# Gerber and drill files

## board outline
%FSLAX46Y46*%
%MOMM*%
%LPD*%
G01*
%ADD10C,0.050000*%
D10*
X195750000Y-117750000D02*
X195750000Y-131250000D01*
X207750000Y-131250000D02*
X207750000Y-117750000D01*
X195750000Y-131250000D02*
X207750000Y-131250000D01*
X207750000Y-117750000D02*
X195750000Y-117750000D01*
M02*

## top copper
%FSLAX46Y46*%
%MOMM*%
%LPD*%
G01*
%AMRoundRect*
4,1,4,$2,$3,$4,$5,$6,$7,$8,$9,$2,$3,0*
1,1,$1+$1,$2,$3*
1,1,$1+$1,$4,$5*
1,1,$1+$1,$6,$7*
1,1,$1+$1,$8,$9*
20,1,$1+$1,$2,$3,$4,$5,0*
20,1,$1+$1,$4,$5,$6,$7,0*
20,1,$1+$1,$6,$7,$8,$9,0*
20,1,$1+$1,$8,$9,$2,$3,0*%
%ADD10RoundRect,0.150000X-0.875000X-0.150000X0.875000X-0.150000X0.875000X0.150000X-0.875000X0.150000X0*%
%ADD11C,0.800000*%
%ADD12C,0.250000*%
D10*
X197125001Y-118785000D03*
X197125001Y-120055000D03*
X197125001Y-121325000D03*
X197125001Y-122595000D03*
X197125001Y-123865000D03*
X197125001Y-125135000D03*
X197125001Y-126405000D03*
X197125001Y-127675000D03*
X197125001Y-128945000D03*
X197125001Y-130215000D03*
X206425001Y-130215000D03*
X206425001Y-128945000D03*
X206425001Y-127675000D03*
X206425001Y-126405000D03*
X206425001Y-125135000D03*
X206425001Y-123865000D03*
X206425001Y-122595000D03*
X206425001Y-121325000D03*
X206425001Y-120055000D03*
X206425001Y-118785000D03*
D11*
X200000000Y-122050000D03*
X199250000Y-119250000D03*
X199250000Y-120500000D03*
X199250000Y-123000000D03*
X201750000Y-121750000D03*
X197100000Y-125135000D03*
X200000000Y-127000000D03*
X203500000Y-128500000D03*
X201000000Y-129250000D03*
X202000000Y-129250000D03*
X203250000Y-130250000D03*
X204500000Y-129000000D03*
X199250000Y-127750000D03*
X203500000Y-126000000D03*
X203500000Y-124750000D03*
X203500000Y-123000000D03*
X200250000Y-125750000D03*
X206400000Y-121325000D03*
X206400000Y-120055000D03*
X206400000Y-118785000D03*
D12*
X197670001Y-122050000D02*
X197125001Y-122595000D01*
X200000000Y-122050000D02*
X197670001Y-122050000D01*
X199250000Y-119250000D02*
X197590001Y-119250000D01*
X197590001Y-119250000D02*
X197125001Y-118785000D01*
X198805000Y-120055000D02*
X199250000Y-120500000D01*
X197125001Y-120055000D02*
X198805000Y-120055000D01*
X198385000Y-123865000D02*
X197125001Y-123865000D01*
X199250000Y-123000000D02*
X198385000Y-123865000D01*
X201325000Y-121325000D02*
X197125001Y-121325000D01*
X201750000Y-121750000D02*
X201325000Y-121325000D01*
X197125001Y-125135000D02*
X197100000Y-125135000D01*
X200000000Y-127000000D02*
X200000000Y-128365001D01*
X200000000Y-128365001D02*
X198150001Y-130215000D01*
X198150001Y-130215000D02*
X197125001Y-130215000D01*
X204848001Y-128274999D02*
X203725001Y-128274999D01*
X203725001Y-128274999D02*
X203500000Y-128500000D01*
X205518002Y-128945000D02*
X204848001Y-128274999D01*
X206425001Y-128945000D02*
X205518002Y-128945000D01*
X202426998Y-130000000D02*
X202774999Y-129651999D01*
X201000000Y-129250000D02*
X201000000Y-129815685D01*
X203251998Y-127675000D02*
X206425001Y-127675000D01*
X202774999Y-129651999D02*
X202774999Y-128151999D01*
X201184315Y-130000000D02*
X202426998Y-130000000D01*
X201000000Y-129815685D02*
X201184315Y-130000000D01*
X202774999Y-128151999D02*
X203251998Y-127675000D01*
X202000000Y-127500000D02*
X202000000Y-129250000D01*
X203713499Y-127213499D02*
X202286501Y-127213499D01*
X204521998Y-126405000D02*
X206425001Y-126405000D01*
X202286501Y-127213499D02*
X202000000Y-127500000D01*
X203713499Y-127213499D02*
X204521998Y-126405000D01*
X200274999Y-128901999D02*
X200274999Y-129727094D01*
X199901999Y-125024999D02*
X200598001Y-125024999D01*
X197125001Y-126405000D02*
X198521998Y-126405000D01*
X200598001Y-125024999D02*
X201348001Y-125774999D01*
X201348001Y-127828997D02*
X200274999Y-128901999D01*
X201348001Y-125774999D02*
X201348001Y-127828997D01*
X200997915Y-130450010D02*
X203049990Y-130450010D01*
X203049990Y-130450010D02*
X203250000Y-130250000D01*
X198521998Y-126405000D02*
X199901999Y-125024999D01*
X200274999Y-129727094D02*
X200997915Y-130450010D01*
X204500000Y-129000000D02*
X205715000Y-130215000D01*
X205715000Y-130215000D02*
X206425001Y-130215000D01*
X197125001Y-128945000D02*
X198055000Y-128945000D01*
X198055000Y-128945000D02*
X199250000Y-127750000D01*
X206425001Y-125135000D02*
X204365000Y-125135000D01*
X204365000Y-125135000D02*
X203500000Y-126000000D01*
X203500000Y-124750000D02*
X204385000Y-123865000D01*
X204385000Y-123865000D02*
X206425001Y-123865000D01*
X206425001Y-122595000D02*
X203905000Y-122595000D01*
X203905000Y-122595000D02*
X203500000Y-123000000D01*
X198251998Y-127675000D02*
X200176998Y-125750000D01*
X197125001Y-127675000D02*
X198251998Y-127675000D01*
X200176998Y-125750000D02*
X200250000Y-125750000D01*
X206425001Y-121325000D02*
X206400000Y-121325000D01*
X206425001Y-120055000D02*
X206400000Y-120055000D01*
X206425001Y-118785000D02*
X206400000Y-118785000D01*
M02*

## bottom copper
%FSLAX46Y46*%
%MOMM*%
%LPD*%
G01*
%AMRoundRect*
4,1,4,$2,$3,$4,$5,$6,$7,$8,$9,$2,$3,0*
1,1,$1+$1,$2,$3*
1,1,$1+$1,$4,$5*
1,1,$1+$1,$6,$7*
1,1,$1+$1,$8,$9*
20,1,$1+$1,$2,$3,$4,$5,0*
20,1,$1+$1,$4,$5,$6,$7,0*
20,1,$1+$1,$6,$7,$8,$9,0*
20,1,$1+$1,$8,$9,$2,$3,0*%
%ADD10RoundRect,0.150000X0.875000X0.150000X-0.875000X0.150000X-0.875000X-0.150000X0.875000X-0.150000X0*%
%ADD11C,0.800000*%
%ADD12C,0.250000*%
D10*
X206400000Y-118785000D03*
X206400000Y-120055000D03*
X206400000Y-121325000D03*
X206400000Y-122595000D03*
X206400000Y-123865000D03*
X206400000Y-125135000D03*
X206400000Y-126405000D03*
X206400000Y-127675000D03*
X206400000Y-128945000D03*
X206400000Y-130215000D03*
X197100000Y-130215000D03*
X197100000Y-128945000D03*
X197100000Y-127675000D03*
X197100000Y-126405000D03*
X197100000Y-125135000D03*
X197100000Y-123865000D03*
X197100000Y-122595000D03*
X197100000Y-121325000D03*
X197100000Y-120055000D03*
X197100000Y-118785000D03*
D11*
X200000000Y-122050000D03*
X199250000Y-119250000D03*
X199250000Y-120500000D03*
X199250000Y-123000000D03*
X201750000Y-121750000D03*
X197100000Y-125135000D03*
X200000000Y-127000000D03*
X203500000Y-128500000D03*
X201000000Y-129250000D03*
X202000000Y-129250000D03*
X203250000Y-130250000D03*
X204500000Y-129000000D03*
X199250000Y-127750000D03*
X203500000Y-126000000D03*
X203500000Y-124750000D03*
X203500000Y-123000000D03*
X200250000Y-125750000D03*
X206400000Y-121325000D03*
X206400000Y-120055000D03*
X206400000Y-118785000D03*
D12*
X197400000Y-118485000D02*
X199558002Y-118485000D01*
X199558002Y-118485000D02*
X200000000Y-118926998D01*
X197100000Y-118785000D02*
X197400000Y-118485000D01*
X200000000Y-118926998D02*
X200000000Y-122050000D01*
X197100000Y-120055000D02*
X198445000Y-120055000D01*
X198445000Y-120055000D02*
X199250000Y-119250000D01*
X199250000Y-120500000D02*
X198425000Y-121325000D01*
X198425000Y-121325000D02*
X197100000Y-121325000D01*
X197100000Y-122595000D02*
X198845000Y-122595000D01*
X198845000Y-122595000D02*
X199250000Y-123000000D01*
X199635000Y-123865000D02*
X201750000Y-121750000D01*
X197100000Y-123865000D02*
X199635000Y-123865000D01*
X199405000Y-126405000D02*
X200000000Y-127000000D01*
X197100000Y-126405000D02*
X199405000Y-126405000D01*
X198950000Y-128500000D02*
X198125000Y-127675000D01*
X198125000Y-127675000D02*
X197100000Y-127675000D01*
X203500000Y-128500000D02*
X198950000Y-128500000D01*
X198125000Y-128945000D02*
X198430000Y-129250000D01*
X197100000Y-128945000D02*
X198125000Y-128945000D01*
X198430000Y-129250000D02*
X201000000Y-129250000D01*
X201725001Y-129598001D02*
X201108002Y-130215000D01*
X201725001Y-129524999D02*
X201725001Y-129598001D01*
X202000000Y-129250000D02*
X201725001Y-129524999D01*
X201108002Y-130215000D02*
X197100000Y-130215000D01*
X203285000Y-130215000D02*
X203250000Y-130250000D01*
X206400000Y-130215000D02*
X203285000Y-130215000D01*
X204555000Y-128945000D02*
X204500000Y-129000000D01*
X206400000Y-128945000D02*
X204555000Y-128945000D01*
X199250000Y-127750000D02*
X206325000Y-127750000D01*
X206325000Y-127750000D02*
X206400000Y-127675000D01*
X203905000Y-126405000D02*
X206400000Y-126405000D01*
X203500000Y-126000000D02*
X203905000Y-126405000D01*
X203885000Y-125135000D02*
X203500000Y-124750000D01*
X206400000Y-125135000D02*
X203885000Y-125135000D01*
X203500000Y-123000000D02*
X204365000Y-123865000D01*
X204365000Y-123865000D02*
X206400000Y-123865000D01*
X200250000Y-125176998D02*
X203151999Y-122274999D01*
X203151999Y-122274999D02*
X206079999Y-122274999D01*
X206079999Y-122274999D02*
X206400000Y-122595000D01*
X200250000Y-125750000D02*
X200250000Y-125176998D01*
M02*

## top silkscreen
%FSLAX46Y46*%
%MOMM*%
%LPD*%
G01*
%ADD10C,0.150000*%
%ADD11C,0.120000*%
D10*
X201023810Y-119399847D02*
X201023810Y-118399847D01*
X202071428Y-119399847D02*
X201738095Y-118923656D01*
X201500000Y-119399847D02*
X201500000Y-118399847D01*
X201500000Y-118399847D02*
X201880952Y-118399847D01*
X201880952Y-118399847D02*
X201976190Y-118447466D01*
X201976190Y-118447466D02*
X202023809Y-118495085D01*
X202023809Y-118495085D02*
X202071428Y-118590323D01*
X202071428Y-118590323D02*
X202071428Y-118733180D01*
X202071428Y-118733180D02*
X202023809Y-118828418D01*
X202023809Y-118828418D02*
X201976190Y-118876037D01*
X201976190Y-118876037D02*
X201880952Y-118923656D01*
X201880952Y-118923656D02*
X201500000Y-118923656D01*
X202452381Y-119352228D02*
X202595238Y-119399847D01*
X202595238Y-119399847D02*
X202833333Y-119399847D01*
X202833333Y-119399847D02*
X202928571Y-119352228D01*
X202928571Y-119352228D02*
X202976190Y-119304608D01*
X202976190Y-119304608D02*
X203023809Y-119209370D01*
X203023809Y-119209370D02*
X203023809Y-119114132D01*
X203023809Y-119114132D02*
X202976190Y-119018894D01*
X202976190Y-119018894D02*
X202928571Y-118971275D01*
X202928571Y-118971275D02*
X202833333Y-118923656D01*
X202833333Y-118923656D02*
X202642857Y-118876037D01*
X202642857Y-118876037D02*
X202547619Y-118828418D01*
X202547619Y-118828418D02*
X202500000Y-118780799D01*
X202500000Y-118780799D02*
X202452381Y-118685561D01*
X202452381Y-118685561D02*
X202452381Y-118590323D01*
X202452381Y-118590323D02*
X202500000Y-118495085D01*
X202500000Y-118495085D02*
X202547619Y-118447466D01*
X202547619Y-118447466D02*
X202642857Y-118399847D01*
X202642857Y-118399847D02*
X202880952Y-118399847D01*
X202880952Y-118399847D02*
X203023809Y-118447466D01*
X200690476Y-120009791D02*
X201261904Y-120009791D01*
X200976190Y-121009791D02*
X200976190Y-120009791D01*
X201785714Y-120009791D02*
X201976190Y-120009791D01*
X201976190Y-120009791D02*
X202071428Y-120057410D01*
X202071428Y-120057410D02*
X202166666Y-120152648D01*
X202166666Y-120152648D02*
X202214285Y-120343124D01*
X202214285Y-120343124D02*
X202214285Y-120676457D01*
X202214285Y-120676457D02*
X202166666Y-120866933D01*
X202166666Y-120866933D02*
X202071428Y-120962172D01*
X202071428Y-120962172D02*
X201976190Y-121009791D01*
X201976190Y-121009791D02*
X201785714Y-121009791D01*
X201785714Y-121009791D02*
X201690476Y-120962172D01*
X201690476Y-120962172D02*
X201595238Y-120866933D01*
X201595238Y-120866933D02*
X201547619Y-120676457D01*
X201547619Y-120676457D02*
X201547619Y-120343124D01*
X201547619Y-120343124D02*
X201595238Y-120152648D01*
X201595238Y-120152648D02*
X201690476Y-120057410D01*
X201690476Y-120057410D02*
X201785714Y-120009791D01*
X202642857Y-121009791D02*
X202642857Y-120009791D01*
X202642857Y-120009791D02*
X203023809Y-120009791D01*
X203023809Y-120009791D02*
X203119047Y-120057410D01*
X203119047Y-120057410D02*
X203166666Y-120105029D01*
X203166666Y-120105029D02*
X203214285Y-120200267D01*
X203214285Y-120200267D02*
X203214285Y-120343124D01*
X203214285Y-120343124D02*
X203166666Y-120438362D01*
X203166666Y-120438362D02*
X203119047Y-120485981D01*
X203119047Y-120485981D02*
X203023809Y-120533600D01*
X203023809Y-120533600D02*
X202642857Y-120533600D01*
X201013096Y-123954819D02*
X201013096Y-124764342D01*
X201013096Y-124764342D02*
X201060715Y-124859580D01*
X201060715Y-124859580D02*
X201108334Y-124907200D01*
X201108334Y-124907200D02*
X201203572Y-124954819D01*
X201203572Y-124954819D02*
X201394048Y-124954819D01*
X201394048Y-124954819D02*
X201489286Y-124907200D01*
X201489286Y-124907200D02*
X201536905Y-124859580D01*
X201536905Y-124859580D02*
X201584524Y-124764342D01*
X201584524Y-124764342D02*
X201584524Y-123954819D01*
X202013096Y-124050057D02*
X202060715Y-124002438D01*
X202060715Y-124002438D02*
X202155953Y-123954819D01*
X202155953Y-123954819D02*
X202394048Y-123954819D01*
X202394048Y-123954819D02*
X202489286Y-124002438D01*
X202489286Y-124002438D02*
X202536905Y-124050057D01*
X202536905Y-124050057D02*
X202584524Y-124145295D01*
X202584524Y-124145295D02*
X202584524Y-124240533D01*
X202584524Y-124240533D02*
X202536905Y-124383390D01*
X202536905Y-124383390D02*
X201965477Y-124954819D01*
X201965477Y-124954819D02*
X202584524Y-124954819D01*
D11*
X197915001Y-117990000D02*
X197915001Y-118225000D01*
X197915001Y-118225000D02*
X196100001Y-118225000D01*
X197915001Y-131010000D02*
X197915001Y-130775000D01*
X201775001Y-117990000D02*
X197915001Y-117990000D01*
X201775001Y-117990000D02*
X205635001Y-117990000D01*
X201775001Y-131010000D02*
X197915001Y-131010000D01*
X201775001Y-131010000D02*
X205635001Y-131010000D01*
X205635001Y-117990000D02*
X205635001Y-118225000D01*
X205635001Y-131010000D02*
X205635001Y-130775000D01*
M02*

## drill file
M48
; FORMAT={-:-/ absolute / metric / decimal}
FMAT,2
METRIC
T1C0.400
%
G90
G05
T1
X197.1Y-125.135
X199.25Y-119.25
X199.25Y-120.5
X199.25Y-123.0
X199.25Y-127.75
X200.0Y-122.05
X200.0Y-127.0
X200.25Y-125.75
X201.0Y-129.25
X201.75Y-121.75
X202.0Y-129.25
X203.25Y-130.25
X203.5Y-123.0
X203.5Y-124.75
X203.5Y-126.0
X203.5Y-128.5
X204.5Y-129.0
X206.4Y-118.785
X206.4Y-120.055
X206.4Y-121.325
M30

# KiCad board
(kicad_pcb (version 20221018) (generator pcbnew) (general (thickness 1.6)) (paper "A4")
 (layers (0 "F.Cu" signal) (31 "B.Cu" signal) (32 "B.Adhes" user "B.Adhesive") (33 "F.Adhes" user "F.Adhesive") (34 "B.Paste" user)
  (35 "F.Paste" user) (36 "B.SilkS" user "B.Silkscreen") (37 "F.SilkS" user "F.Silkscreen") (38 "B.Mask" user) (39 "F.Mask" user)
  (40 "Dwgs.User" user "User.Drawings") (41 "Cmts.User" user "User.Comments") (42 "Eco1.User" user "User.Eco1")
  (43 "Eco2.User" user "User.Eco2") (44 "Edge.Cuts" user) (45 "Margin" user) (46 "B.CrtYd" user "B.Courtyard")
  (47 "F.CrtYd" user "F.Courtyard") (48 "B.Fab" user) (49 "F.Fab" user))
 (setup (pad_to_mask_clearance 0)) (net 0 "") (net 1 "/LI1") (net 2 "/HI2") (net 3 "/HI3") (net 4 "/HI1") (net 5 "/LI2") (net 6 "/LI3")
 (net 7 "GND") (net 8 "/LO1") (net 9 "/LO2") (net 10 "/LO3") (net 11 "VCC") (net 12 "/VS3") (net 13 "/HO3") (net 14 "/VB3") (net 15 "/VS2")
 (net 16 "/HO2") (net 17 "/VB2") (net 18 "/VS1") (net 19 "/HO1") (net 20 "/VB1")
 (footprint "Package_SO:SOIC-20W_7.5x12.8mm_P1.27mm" (layer "F.Cu") (at 201.775001 124.5)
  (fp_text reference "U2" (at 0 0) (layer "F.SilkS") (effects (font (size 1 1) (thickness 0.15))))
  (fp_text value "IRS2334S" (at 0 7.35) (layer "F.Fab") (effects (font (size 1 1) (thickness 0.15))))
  (fp_line (start -3.86 -6.51) (end -3.86 -6.275) (stroke (width 0.12) (type solid)) (layer "F.SilkS"))
  (fp_line (start -3.86 -6.275) (end -5.675 -6.275) (stroke (width 0.12) (type solid)) (layer "F.SilkS"))
  (fp_line (start -3.86 6.51) (end -3.86 6.275) (stroke (width 0.12) (type solid)) (layer "F.SilkS"))
  (fp_line (start 0 -6.51) (end -3.86 -6.51) (stroke (width 0.12) (type solid)) (layer "F.SilkS"))
  (fp_line (start 0 -6.51) (end 3.86 -6.51) (stroke (width 0.12) (type solid)) (layer "F.SilkS"))
  (fp_line (start 0 6.51) (end -3.86 6.51) (stroke (width 0.12) (type solid)) (layer "F.SilkS"))
  (fp_line (start 0 6.51) (end 3.86 6.51) (stroke (width 0.12) (type solid)) (layer "F.SilkS"))
  (fp_line (start 3.86 -6.51) (end 3.86 -6.275) (stroke (width 0.12) (type solid)) (layer "F.SilkS"))
  (fp_line (start 3.86 6.51) (end 3.86 6.275) (stroke (width 0.12) (type solid)) (layer "F.SilkS"))
  (pad "1" smd roundrect (at -4.65 -5.715) (size 2.05 0.6) (layers "F.Cu" "F.Paste" "F.Mask") (roundrect_rratio 0.25) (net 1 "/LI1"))
  (pad "2" smd roundrect (at -4.65 -4.445) (size 2.05 0.6) (layers "F.Cu" "F.Paste" "F.Mask") (roundrect_rratio 0.25) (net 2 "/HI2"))
  (pad "3" smd roundrect (at -4.65 -3.175) (size 2.05 0.6) (layers "F.Cu" "F.Paste" "F.Mask") (roundrect_rratio 0.25) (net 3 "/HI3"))
  (pad "4" smd roundrect (at -4.65 -1.905) (size 2.05 0.6) (layers "F.Cu" "F.Paste" "F.Mask") (roundrect_rratio 0.25) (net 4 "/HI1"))
  (pad "5" smd roundrect (at -4.65 -0.635) (size 2.05 0.6) (layers "F.Cu" "F.Paste" "F.Mask") (roundrect_rratio 0.25) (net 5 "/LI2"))
  (pad "6" smd roundrect (at -4.65 0.635) (size 2.05 0.6) (layers "F.Cu" "F.Paste" "F.Mask") (roundrect_rratio 0.25) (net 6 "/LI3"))
  (pad "7" smd roundrect (at -4.65 1.905) (size 2.05 0.6) (layers "F.Cu" "F.Paste" "F.Mask") (roundrect_rratio 0.25) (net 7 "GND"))
  (pad "8" smd roundrect (at -4.65 3.175) (size 2.05 0.6) (layers "F.Cu" "F.Paste" "F.Mask") (roundrect_rratio 0.25) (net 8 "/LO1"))
  (pad "9" smd roundrect (at -4.65 4.445) (size 2.05 0.6) (layers "F.Cu" "F.Paste" "F.Mask") (roundrect_rratio 0.25) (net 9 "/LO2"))
  (pad "10" smd roundrect (at -4.65 5.715) (size 2.05 0.6) (layers "F.Cu" "F.Paste" "F.Mask") (roundrect_rratio 0.25) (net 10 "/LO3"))
  (pad "11" smd roundrect (at 4.65 5.715) (size 2.05 0.6) (layers "F.Cu" "F.Paste" "F.Mask") (roundrect_rratio 0.25) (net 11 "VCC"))
  (pad "12" smd roundrect (at 4.65 4.445) (size 2.05 0.6) (layers "F.Cu" "F.Paste" "F.Mask") (roundrect_rratio 0.25) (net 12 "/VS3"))
  (pad "13" smd roundrect (at 4.65 3.175) (size 2.05 0.6) (layers "F.Cu" "F.Paste" "F.Mask") (roundrect_rratio 0.25) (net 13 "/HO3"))
  (pad "14" smd roundrect (at 4.65 1.905) (size 2.05 0.6) (layers "F.Cu" "F.Paste" "F.Mask") (roundrect_rratio 0.25) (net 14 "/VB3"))
  (pad "15" smd roundrect (at 4.65 0.635) (size 2.05 0.6) (layers "F.Cu" "F.Paste" "F.Mask") (roundrect_rratio 0.25) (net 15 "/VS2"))
  (pad "16" smd roundrect (at 4.65 -0.635) (size 2.05 0.6) (layers "F.Cu" "F.Paste" "F.Mask") (roundrect_rratio 0.25) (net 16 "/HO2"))
  (pad "17" smd roundrect (at 4.65 -1.905) (size 2.05 0.6) (layers "F.Cu" "F.Paste" "F.Mask") (roundrect_rratio 0.25) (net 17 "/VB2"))
  (pad "18" smd roundrect (at 4.65 -3.175) (size 2.05 0.6) (layers "F.Cu" "F.Paste" "F.Mask") (roundrect_rratio 0.25) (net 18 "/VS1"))
  (pad "19" smd roundrect (at 4.65 -4.445) (size 2.05 0.6) (layers "F.Cu" "F.Paste" "F.Mask") (roundrect_rratio 0.25) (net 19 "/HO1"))
  (pad "20" smd roundrect (at 4.65 -5.715) (size 2.05 0.6) (layers "F.Cu" "F.Paste" "F.Mask") (roundrect_rratio 0.25) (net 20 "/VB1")))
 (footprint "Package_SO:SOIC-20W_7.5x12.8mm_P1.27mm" (layer "B.Cu") (at 201.75 124.5 180)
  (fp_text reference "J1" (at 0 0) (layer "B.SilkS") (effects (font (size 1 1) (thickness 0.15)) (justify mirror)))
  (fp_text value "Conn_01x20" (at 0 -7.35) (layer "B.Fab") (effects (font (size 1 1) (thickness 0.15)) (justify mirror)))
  (pad "1" smd roundrect (at -4.65 5.715 180) (size 2.05 0.6) (layers "B.Cu" "B.Paste" "B.Mask") (roundrect_rratio 0.25) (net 20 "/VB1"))
  (pad "2" smd roundrect (at -4.65 4.445 180) (size 2.05 0.6) (layers "B.Cu" "B.Paste" "B.Mask") (roundrect_rratio 0.25) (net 19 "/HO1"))
  (pad "3" smd roundrect (at -4.65 3.175 180) (size 2.05 0.6) (layers "B.Cu" "B.Paste" "B.Mask") (roundrect_rratio 0.25) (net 18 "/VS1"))
  (pad "4" smd roundrect (at -4.65 1.905 180) (size 2.05 0.6) (layers "B.Cu" "B.Paste" "B.Mask") (roundrect_rratio 0.25) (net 8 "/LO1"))
  (pad "5" smd roundrect (at -4.65 0.635 180) (size 2.05 0.6) (layers "B.Cu" "B.Paste" "B.Mask") (roundrect_rratio 0.25) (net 17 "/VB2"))
  (pad "6" smd roundrect (at -4.65 -0.635 180) (size 2.05 0.6) (layers "B.Cu" "B.Paste" "B.Mask") (roundrect_rratio 0.25) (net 16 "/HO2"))
  (pad "7" smd roundrect (at -4.65 -1.905 180) (size 2.05 0.6) (layers "B.Cu" "B.Paste" "B.Mask") (roundrect_rratio 0.25) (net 15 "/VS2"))
  (pad "8" smd roundrect (at -4.65 -3.175 180) (size 2.05 0.6) (layers "B.Cu" "B.Paste" "B.Mask") (roundrect_rratio 0.25) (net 9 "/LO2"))
  (pad "9" smd roundrect (at -4.65 -4.445 180) (size 2.05 0.6) (layers "B.Cu" "B.Paste" "B.Mask") (roundrect_rratio 0.25) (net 11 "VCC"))
  (pad "10" smd roundrect (at -4.65 -5.715 180) (size 2.05 0.6) (layers "B.Cu" "B.Paste" "B.Mask") (roundrect_rratio 0.25) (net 7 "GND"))
  (pad "11" smd roundrect (at 4.65 -5.715 180) (size 2.05 0.6) (layers "B.Cu" "B.Paste" "B.Mask") (roundrect_rratio 0.25) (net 14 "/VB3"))
  (pad "12" smd roundrect (at 4.65 -4.445 180) (size 2.05 0.6) (layers "B.Cu" "B.Paste" "B.Mask") (roundrect_rratio 0.25) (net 13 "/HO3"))
  (pad "13" smd roundrect (at 4.65 -3.175 180) (size 2.05 0.6) (layers "B.Cu" "B.Paste" "B.Mask") (roundrect_rratio 0.25) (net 12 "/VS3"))
  (pad "14" smd roundrect (at 4.65 -1.905 180) (size 2.05 0.6) (layers "B.Cu" "B.Paste" "B.Mask") (roundrect_rratio 0.25) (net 10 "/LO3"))
  (pad "15" smd roundrect (at 4.65 -0.635 180) (size 2.05 0.6) (layers "B.Cu" "B.Paste" "B.Mask") (roundrect_rratio 0.25) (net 6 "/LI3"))
  (pad "16" smd roundrect (at 4.65 0.635 180) (size 2.05 0.6) (layers "B.Cu" "B.Paste" "B.Mask") (roundrect_rratio 0.25) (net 3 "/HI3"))
  (pad "17" smd roundrect (at 4.65 1.905 180) (size 2.05 0.6) (layers "B.Cu" "B.Paste" "B.Mask") (roundrect_rratio 0.25) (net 5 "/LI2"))
  (pad "18" smd roundrect (at 4.65 3.175 180) (size 2.05 0.6) (layers "B.Cu" "B.Paste" "B.Mask") (roundrect_rratio 0.25) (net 2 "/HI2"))
  (pad "19" smd roundrect (at 4.65 4.445 180) (size 2.05 0.6) (layers "B.Cu" "B.Paste" "B.Mask") (roundrect_rratio 0.25) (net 1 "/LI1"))
  (pad "20" smd roundrect (at 4.65 5.715 180) (size 2.05 0.6) (layers "B.Cu" "B.Paste" "B.Mask") (roundrect_rratio 0.25) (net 4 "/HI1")))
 (gr_line (start 195.75 117.75) (end 195.75 131.25) (stroke (width 0.05) (type solid)) (layer "Edge.Cuts"))
 (gr_line (start 207.75 131.25) (end 207.75 117.75) (stroke (width 0.05) (type solid)) (layer "Edge.Cuts"))
 (gr_line (start 195.75 131.25) (end 207.75 131.25) (stroke (width 0.05) (type solid)) (layer "Edge.Cuts"))
 (gr_line (start 207.75 117.75) (end 195.75 117.75) (stroke (width 0.05) (type solid)) (layer "Edge.Cuts"))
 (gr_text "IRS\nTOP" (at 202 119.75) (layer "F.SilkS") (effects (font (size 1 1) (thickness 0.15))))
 (segment (start 197.670001 122.05) (end 197.125001 122.595) (width 0.25) (layer "F.Cu") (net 4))
 (segment (start 200 122.05) (end 197.670001 122.05) (width 0.25) (layer "F.Cu") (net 4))
 (via (at 200 122.05) (size 0.8) (drill 0.4) (layers "F.Cu" "B.Cu") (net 4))
 (segment (start 197.4 118.485) (end 199.558002 118.485) (width 0.25) (layer "B.Cu") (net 4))
 (segment (start 199.558002 118.485) (end 200 118.926998) (width 0.25) (layer "B.Cu") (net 4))
 (segment (start 197.1 118.785) (end 197.4 118.485) (width 0.25) (layer "B.Cu") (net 4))
 (segment (start 200 118.926998) (end 200 122.05) (width 0.25) (layer "B.Cu") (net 4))
 (segment (start 199.25 119.25) (end 197.590001 119.25) (width 0.25) (layer "F.Cu") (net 1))
 (segment (start 197.590001 119.25) (end 197.125001 118.785) (width 0.25) (layer "F.Cu") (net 1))
 (via (at 199.25 119.25) (size 0.8) (drill 0.4) (layers "F.Cu" "B.Cu") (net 1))
 (segment (start 197.1 120.055) (end 198.445 120.055) (width 0.25) (layer "B.Cu") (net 1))
 (segment (start 198.445 120.055) (end 199.25 119.25) (width 0.25) (layer "B.Cu") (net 1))
 (segment (start 198.805 120.055) (end 199.25 120.5) (width 0.25) (layer "F.Cu") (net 2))
 (segment (start 197.125001 120.055) (end 198.805 120.055) (width 0.25) (layer "F.Cu") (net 2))
 (via (at 199.25 120.5) (size 0.8) (drill 0.4) (layers "F.Cu" "B.Cu") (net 2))
 (segment (start 199.25 120.5) (end 198.425 121.325) (width 0.25) (layer "B.Cu") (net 2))
 (segment (start 198.425 121.325) (end 197.1 121.325) (width 0.25) (layer "B.Cu") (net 2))
 (segment (start 198.385 123.865) (end 197.125001 123.865) (width 0.25) (layer "F.Cu") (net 5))
 (segment (start 199.25 123) (end 198.385 123.865) (width 0.25) (layer "F.Cu") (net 5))
 (via (at 199.25 123) (size 0.8) (drill 0.4) (layers "F.Cu" "B.Cu") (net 5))
 (segment (start 197.1 122.595) (end 198.845 122.595) (width 0.25) (layer "B.Cu") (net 5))
 (segment (start 198.845 122.595) (end 199.25 123) (width 0.25) (layer "B.Cu") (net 5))
 (segment (start 201.325 121.325) (end 197.125001 121.325) (width 0.25) (layer "F.Cu") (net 3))
 (segment (start 201.75 121.75) (end 201.325 121.325) (width 0.25) (layer "F.Cu") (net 3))
 (via (at 201.75 121.75) (size 0.8) (drill 0.4) (layers "F.Cu" "B.Cu") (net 3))
 (segment (start 199.635 123.865) (end 201.75 121.75) (width 0.25) (layer "B.Cu") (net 3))
 (segment (start 197.1 123.865) (end 199.635 123.865) (width 0.25) (layer "B.Cu") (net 3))
 (segment (start 197.125001 125.135) (end 197.1 125.135) (width 0.25) (layer "F.Cu") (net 6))
 (via (at 197.1 125.135) (size 0.8) (drill 0.4) (layers "F.Cu" "B.Cu") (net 6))
 (segment (start 200 127) (end 200 128.365001) (width 0.25) (layer "F.Cu") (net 10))
 (segment (start 200 128.365001) (end 198.150001 130.215) (width 0.25) (layer "F.Cu") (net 10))
 (segment (start 198.150001 130.215) (end 197.125001 130.215) (width 0.25) (layer "F.Cu") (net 10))
 (via (at 200 127) (size 0.8) (drill 0.4) (layers "F.Cu" "B.Cu") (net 10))
 (segment (start 199.405 126.405) (end 200 127) (width 0.25) (layer "B.Cu") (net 10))
 (segment (start 197.1 126.405) (end 199.405 126.405) (width 0.25) (layer "B.Cu") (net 10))
 (segment (start 204.848001 128.274999) (end 203.725001 128.274999) (width 0.25) (layer "F.Cu") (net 12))
 (segment (start 203.725001 128.274999) (end 203.5 128.5) (width 0.25) (layer "F.Cu") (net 12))
 (segment (start 205.518002 128.945) (end 204.848001 128.274999) (width 0.25) (layer "F.Cu") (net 12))
 (segment (start 206.425001 128.945) (end 205.518002 128.945) (width 0.25) (layer "F.Cu") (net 12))
 (via (at 203.5 128.5) (size 0.8) (drill 0.4) (layers "F.Cu" "B.Cu") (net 12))
 (segment (start 198.95 128.5) (end 198.125 127.675) (width 0.25) (layer "B.Cu") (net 12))
 (segment (start 198.125 127.675) (end 197.1 127.675) (width 0.25) (layer "B.Cu") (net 12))
 (segment (start 203.5 128.5) (end 198.95 128.5) (width 0.25) (layer "B.Cu") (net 12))
 (segment (start 202.426998 130) (end 202.774999 129.651999) (width 0.25) (layer "F.Cu") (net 13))
 (segment (start 201 129.25) (end 201 129.815685) (width 0.25) (layer "F.Cu") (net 13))
 (segment (start 203.251998 127.675) (end 206.425001 127.675) (width 0.25) (layer "F.Cu") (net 13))
 (segment (start 202.774999 129.651999) (end 202.774999 128.151999) (width 0.25) (layer "F.Cu") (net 13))
 (segment (start 201.184315 130) (end 202.426998 130) (width 0.25) (layer "F.Cu") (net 13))
 (segment (start 201 129.815685) (end 201.184315 130) (width 0.25) (layer "F.Cu") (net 13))
 (segment (start 202.774999 128.151999) (end 203.251998 127.675) (width 0.25) (layer "F.Cu") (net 13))
 (via (at 201 129.25) (size 0.8) (drill 0.4) (layers "F.Cu" "B.Cu") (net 13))
 (segment (start 198.125 128.945) (end 198.43 129.25) (width 0.25) (layer "B.Cu") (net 13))
 (segment (start 197.1 128.945) (end 198.125 128.945) (width 0.25) (layer "B.Cu") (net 13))
 (segment (start 198.43 129.25) (end 201 129.25) (width 0.25) (layer "B.Cu") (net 13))
 (segment (start 202 127.5) (end 202 129.25) (width 0.25) (layer "F.Cu") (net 14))
 (segment (start 203.713499 127.213499) (end 202.286501 127.213499) (width 0.25) (layer "F.Cu") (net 14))
 (segment (start 204.521998 126.405) (end 206.425001 126.405) (width 0.25) (layer "F.Cu") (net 14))
 (segment (start 202.286501 127.213499) (end 202 127.5) (width 0.25) (layer "F.Cu") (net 14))
 (segment (start 203.713499 127.213499) (end 204.521998 126.405) (width 0.25) (layer "F.Cu") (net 14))
 (via (at 202 129.25) (size 0.8) (drill 0.4) (layers "F.Cu" "B.Cu") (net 14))
 (segment (start 201.725001 129.598001) (end 201.108002 130.215) (width 0.25) (layer "B.Cu") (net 14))
 (segment (start 201.725001 129.524999) (end 201.725001 129.598001) (width 0.25) (layer "B.Cu") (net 14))
 (segment (start 202 129.25) (end 201.725001 129.524999) (width 0.25) (layer "B.Cu") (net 14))
 (segment (start 201.108002 130.215) (end 197.1 130.215) (width 0.25) (layer "B.Cu") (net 14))
 (segment (start 200.274999 128.901999) (end 200.274999 129.727094) (width 0.25) (layer "F.Cu") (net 7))
 (segment (start 199.901999 125.024999) (end 200.598001 125.024999) (width 0.25) (layer "F.Cu") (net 7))
 (segment (start 197.125001 126.405) (end 198.521998 126.405) (width 0.25) (layer "F.Cu") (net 7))
 (segment (start 200.598001 125.024999) (end 201.348001 125.774999) (width 0.25) (layer "F.Cu") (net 7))
 (segment (start 201.348001 127.828997) (end 200.274999 128.901999) (width 0.25) (layer "F.Cu") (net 7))
 (segment (start 201.348001 125.774999) (end 201.348001 127.828997) (width 0.25) (layer "F.Cu") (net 7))
 (segment (start 200.997915 130.45001) (end 203.04999 130.45001) (width 0.25) (layer "F.Cu") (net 7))
 (segment (start 203.04999 130.45001) (end 203.25 130.25) (width 0.25) (layer "F.Cu") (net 7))
 (segment (start 198.521998 126.405) (end 199.901999 125.024999) (width 0.25) (layer "F.Cu") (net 7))
 (segment (start 200.274999 129.727094) (end 200.997915 130.45001) (width 0.25) (layer "F.Cu") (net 7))
 (via (at 203.25 130.25) (size 0.8) (drill 0.4) (layers "F.Cu" "B.Cu") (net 7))
 (segment (start 203.285 130.215) (end 203.25 130.25) (width 0.25) (layer "B.Cu") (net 7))
 (segment (start 206.4 130.215) (end 203.285 130.215) (width 0.25) (layer "B.Cu") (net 7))
 (segment (start 204.5 129) (end 205.715 130.215) (width 0.25) (layer "F.Cu") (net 11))
 (segment (start 205.715 130.215) (end 206.425001 130.215) (width 0.25) (layer "F.Cu") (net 11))
 (via (at 204.5 129) (size 0.8) (drill 0.4) (layers "F.Cu" "B.Cu") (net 11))
 (segment (start 204.555 128.945) (end 204.5 129) (width 0.25) (layer "B.Cu") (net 11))
 (segment (start 206.4 128.945) (end 204.555 128.945) (width 0.25) (layer "B.Cu") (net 11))
 (segment (start 197.125001 128.945) (end 198.055 128.945) (width 0.25) (layer "F.Cu") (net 9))
 (segment (start 198.055 128.945) (end 199.25 127.75) (width 0.25) (layer "F.Cu") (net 9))
 (via (at 199.25 127.75) (size 0.8) (drill 0.4) (layers "F.Cu" "B.Cu") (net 9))
 (segment (start 199.25 127.75) (end 206.325 127.75) (width 0.25) (layer "B.Cu") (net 9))
 (segment (start 206.325 127.75) (end 206.4 127.675) (width 0.25) (layer "B.Cu") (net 9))
 (segment (start 206.425001 125.135) (end 204.365 125.135) (width 0.25) (layer "F.Cu") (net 15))
 (segment (start 204.365 125.135) (end 203.5 126) (width 0.25) (layer "F.Cu") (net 15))
 (via (at 203.5 126) (size 0.8) (drill 0.4) (layers "F.Cu" "B.Cu") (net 15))
 (segment (start 203.905 126.405) (end 206.4 126.405) (width 0.25) (layer "B.Cu") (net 15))
 (segment (start 203.5 126) (end 203.905 126.405) (width 0.25) (layer "B.Cu") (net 15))
 (segment (start 203.5 124.75) (end 204.385 123.865) (width 0.25) (layer "F.Cu") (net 16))
 (segment (start 204.385 123.865) (end 206.425001 123.865) (width 0.25) (layer "F.Cu") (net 16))
 (via (at 203.5 124.75) (size 0.8) (drill 0.4) (layers "F.Cu" "B.Cu") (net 16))
 (segment (start 203.885 125.135) (end 203.5 124.75) (width 0.25) (layer "B.Cu") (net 16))
 (segment (start 206.4 125.135) (end 203.885 125.135) (width 0.25) (layer "B.Cu") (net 16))
 (segment (start 206.425001 122.595) (end 203.905 122.595) (width 0.25) (layer "F.Cu") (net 17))
 (segment (start 203.905 122.595) (end 203.5 123) (width 0.25) (layer "F.Cu") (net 17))
 (via (at 203.5 123) (size 0.8) (drill 0.4) (layers "F.Cu" "B.Cu") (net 17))
 (segment (start 203.5 123) (end 204.365 123.865) (width 0.25) (layer "B.Cu") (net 17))
 (segment (start 204.365 123.865) (end 206.4 123.865) (width 0.25) (layer "B.Cu") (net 17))
 (segment (start 198.251998 127.675) (end 200.176998 125.75) (width 0.25) (layer "F.Cu") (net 8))
 (segment (start 197.125001 127.675) (end 198.251998 127.675) (width 0.25) (layer "F.Cu") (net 8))
 (segment (start 200.176998 125.75) (end 200.25 125.75) (width 0.25) (layer "F.Cu") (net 8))
 (via (at 200.25 125.75) (size 0.8) (drill 0.4) (layers "F.Cu" "B.Cu") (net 8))
 (segment (start 200.25 125.176998) (end 203.151999 122.274999) (width 0.25) (layer "B.Cu") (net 8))
 (segment (start 203.151999 122.274999) (end 206.079999 122.274999) (width 0.25) (layer "B.Cu") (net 8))
 (segment (start 206.079999 122.274999) (end 206.4 122.595) (width 0.25) (layer "B.Cu") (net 8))
 (segment (start 200.25 125.75) (end 200.25 125.176998) (width 0.25) (layer "B.Cu") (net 8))
 (segment (start 206.425001 121.325) (end 206.4 121.325) (width 0.25) (layer "F.Cu") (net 18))
 (via (at 206.4 121.325) (size 0.8) (drill 0.4) (layers "F.Cu" "B.Cu") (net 18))
 (segment (start 206.425001 120.055) (end 206.4 120.055) (width 0.25) (layer "F.Cu") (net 19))
 (via (at 206.4 120.055) (size 0.8) (drill 0.4) (layers "F.Cu" "B.Cu") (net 19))
 (segment (start 206.425001 118.785) (end 206.4 118.785) (width 0.25) (layer "F.Cu") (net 20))
 (via (at 206.4 118.785) (size 0.8) (drill 0.4) (layers "F.Cu" "B.Cu") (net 20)))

